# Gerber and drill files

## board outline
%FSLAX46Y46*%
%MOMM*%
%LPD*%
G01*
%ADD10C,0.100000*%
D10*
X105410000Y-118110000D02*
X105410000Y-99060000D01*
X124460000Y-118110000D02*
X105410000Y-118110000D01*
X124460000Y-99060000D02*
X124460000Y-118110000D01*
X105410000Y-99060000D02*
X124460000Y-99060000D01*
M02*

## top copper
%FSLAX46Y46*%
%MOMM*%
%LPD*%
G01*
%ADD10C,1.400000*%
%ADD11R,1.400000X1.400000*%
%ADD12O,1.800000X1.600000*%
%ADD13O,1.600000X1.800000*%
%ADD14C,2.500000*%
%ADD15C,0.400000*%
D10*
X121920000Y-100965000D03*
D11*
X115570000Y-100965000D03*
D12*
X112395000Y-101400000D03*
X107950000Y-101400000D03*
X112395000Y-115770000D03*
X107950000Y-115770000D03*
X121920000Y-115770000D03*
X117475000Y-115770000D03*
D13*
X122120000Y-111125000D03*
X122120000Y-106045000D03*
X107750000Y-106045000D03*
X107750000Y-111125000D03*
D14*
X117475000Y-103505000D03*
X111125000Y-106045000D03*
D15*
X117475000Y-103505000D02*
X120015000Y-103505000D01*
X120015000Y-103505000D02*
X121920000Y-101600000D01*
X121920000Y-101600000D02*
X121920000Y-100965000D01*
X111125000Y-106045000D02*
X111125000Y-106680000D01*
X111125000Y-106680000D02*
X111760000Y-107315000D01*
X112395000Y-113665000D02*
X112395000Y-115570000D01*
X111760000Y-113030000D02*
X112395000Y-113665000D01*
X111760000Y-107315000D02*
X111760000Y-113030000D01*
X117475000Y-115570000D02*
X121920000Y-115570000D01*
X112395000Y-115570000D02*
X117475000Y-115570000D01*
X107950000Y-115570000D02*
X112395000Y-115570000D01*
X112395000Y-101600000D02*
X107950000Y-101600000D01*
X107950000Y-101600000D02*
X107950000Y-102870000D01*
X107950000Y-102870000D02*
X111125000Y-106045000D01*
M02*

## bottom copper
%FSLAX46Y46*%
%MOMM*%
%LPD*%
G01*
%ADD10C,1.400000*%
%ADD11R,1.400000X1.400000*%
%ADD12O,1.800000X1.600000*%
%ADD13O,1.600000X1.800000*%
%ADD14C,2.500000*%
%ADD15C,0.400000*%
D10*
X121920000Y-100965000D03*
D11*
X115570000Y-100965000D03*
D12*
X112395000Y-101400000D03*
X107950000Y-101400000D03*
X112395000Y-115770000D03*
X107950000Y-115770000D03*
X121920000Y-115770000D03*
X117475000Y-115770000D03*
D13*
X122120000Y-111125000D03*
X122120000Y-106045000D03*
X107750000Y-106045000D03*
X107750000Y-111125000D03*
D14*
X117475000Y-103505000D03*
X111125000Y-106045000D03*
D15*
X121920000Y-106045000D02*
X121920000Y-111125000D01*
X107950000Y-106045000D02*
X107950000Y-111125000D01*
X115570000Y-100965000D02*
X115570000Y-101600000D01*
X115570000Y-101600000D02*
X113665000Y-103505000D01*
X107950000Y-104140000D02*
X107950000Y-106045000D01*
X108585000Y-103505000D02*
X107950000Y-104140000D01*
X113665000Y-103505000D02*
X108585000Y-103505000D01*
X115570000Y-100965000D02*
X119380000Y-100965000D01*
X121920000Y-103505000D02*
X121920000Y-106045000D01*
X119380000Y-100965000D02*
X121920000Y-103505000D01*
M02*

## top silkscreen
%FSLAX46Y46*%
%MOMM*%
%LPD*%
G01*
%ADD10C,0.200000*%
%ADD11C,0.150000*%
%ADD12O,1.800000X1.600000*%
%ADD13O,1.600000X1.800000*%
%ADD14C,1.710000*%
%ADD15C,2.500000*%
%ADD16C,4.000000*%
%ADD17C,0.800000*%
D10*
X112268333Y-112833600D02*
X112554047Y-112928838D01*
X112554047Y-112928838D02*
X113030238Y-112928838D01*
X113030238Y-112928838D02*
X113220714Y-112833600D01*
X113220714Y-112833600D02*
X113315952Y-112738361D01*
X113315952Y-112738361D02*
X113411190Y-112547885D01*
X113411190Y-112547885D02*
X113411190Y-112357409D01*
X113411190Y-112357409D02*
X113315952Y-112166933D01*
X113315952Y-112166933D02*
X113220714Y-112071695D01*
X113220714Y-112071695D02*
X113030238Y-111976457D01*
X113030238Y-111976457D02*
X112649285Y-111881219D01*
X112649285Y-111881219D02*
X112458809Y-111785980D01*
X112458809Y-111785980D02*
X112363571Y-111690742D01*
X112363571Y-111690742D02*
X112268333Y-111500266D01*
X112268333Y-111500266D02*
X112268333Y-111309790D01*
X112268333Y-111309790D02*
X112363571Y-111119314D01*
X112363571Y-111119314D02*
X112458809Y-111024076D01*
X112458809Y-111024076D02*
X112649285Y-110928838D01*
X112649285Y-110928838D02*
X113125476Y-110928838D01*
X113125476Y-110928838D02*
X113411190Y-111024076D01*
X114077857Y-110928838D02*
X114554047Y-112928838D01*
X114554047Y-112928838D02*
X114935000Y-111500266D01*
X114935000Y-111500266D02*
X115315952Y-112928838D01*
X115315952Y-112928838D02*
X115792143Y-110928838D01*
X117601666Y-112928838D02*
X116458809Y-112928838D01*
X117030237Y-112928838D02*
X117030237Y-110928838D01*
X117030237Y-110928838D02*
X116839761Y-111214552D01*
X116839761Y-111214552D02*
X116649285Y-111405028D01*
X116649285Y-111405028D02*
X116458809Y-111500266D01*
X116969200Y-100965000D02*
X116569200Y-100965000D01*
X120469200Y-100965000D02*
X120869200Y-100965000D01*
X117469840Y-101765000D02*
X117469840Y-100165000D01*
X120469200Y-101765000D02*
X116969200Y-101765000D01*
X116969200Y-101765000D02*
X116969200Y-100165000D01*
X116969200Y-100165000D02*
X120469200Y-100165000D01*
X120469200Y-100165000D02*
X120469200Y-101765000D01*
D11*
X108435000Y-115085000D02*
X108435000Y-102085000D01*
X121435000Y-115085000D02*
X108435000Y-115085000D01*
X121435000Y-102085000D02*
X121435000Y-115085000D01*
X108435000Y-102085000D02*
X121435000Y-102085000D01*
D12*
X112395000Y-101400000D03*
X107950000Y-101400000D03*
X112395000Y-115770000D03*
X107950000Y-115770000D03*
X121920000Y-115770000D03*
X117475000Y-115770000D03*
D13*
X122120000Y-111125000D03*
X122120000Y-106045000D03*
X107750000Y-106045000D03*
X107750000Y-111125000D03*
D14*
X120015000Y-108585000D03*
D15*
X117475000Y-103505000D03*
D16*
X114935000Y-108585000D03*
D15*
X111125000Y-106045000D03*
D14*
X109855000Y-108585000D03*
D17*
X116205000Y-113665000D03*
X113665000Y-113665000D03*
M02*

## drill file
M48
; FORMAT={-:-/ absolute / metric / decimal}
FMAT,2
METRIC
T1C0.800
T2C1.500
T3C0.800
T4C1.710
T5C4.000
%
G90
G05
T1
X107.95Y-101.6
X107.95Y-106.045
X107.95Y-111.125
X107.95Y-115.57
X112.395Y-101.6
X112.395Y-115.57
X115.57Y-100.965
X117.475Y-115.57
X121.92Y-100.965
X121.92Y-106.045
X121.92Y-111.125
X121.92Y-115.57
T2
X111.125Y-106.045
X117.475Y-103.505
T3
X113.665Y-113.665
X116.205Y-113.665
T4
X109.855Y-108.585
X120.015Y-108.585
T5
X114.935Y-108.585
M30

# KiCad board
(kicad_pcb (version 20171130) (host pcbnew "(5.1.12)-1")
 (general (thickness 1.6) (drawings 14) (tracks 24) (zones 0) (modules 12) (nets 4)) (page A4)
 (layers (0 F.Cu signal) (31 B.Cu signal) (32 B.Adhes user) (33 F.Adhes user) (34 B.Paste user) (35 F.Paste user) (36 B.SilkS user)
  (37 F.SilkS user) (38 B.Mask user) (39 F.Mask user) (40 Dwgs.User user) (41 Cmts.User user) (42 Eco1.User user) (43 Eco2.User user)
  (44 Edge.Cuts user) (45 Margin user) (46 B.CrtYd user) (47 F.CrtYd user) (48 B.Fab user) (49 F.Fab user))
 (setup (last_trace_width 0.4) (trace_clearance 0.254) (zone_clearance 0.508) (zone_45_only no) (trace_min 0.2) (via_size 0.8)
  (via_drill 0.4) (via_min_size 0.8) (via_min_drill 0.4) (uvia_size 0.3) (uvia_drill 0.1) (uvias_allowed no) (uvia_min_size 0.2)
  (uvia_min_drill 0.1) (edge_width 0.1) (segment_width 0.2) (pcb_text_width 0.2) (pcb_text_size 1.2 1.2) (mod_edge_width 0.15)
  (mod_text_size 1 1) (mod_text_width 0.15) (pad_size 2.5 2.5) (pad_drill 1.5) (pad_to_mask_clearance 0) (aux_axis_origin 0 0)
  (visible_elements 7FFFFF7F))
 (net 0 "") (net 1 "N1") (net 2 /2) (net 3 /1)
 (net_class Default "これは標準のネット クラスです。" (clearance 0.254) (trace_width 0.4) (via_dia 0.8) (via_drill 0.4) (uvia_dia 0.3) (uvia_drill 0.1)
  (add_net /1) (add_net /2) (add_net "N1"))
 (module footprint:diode (layer B.Cu) (at 115.57 100.965)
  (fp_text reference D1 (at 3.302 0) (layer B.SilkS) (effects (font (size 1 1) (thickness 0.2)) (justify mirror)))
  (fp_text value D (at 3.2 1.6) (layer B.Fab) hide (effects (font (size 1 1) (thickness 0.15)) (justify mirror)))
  (fp_line (start 1.3992 0) (end 0.9992 0) (layer F.SilkS) (width 0.2))
  (fp_line (start 4.8992 0) (end 5.2992 0) (layer F.SilkS) (width 0.2))
  (fp_line (start 1.89984 0.8) (end 1.89984 -0.8) (layer F.SilkS) (width 0.2))
  (fp_line (start 4.8992 0.8) (end 1.3992 0.8) (layer F.SilkS) (width 0.2))
  (fp_line (start 1.3992 0.8) (end 1.3992 -0.8) (layer F.SilkS) (width 0.2))
  (fp_line (start 1.3992 -0.8) (end 4.8992 -0.8) (layer F.SilkS) (width 0.2))
  (fp_line (start 4.8992 -0.8) (end 4.8992 0.8) (layer F.SilkS) (width 0.2))
  (pad 2 thru_hole circle (at 6.35 0) (size 1.4 1.4) (drill 0.8) (layers *.Cu *.Mask B.SilkS) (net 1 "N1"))
  (pad 1 thru_hole rect (at 0 0) (size 1.4 1.4) (drill 0.8) (layers *.Cu *.Mask B.SilkS) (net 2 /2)))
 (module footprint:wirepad (layer F.Cu) (at 112.395 101.6 180)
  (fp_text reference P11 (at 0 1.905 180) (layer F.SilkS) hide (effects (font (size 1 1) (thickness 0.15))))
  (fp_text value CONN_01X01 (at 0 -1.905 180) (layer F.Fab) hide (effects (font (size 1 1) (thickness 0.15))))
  (pad 1 thru_hole oval (at 0 0 180) (size 1.8 1.6) (drill 0.8 (offset 0 0.2)) (layers *.Cu *.Mask F.SilkS) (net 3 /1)))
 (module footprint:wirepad (layer F.Cu) (at 107.95 101.6 180)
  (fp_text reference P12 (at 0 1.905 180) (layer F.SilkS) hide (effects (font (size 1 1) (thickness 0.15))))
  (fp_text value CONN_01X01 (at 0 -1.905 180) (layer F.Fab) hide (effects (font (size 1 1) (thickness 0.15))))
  (pad 1 thru_hole oval (at 0 0 180) (size 1.8 1.6) (drill 0.8 (offset 0 0.2)) (layers *.Cu *.Mask F.SilkS) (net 3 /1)))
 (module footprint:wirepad (layer F.Cu) (at 112.395 115.57)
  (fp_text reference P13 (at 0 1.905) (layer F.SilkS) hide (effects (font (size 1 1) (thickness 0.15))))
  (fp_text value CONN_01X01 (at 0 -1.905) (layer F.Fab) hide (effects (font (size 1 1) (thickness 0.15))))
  (pad 1 thru_hole oval (at 0 0) (size 1.8 1.6) (drill 0.8 (offset 0 0.2)) (layers *.Cu *.Mask F.SilkS) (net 3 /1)))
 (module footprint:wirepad (layer F.Cu) (at 107.95 115.57)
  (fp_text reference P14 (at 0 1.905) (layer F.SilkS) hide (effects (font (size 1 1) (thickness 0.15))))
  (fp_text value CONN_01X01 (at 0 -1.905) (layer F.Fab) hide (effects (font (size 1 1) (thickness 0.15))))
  (pad 1 thru_hole oval (at 0 0) (size 1.8 1.6) (drill 0.8 (offset 0 0.2)) (layers *.Cu *.Mask F.SilkS) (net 3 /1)))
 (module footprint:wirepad (layer F.Cu) (at 121.92 115.57)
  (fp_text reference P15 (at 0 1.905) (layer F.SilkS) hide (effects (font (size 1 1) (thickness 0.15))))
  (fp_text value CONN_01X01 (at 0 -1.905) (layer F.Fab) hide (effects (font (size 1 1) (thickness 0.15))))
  (pad 1 thru_hole oval (at 0 0) (size 1.8 1.6) (drill 0.8 (offset 0 0.2)) (layers *.Cu *.Mask F.SilkS) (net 3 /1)))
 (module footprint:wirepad (layer F.Cu) (at 117.475 115.57)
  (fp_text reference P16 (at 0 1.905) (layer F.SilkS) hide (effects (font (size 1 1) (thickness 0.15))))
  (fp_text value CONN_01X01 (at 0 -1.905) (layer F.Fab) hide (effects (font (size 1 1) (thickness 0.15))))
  (pad 1 thru_hole oval (at 0 0) (size 1.8 1.6) (drill 0.8 (offset 0 0.2)) (layers *.Cu *.Mask F.SilkS) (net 3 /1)))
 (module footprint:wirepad (layer F.Cu) (at 121.92 111.125 90)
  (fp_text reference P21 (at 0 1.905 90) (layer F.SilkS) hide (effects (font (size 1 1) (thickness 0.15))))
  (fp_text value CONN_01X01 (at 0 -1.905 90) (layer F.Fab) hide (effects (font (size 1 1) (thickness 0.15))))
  (pad 1 thru_hole oval (at 0 0 90) (size 1.8 1.6) (drill 0.8 (offset 0 0.2)) (layers *.Cu *.Mask F.SilkS) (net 2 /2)))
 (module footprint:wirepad (layer F.Cu) (at 121.92 106.045 90)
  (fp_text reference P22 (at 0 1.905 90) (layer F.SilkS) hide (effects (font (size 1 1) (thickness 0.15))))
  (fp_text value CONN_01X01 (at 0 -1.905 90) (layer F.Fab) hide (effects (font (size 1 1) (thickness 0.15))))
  (pad 1 thru_hole oval (at 0 0 90) (size 1.8 1.6) (drill 0.8 (offset 0 0.2)) (layers *.Cu *.Mask F.SilkS) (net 2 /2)))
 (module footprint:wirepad (layer F.Cu) (at 107.95 106.045 270)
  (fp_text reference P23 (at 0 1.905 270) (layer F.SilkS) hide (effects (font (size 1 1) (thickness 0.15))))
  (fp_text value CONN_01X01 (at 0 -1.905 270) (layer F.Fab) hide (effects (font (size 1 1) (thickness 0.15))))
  (pad 1 thru_hole oval (at 0 0 270) (size 1.8 1.6) (drill 0.8 (offset 0 0.2)) (layers *.Cu *.Mask F.SilkS) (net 2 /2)))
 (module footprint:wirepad (layer F.Cu) (at 107.95 111.125 270)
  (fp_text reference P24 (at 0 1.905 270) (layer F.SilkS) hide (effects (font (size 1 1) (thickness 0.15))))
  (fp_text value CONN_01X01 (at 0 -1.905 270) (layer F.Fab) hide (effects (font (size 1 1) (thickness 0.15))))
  (pad 1 thru_hole oval (at 0 0 270) (size 1.8 1.6) (drill 0.8 (offset 0 0.2)) (layers *.Cu *.Mask F.SilkS) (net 2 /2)))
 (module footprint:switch (layer F.Cu) (at 114.935 108.585)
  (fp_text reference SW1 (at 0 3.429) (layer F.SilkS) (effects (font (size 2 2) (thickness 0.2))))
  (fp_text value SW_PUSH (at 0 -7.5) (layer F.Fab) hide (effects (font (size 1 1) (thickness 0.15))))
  (fp_line (start -6.5 6.5) (end -6.5 -6.5) (layer F.SilkS) (width 0.15))
  (fp_line (start 6.5 6.5) (end -6.5 6.5) (layer F.SilkS) (width 0.15))
  (fp_line (start 6.5 -6.5) (end 6.5 6.5) (layer F.SilkS) (width 0.15))
  (fp_line (start -6.5 -6.5) (end 6.5 -6.5) (layer F.SilkS) (width 0.15))
  (pad "" np_thru_hole circle (at 5.08 0) (size 1.71 1.71) (drill 1.71) (layers *.Cu *.Mask F.SilkS))
  (pad 2 thru_hole circle (at 2.54 -5.08) (size 2.5 2.5) (drill 1.5) (layers *.Cu *.Mask F.SilkS) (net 1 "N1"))
  (pad "" np_thru_hole circle (at 0 0) (size 4 4) (drill 4) (layers *.Cu *.Mask F.SilkS))
  (pad 1 thru_hole circle (at -3.81 -2.54) (size 2.5 2.5) (drill 1.5) (layers *.Cu *.Mask F.SilkS) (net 3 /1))
  (pad "" np_thru_hole circle (at -5.08 0) (size 1.71 1.71) (drill 1.71) (layers *.Cu *.Mask F.SilkS))
  (pad "" np_thru_hole circle (at 1.27 5.08) (size 0.8 0.8) (drill 0.8) (layers *.Cu *.Mask F.SilkS))
  (pad "" np_thru_hole circle (at -1.27 5.08) (size 0.8 0.8) (drill 0.8) (layers *.Cu *.Mask F.SilkS)))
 (gr_line (start 105.41 118.11) (end 105.41 99.06) (angle 90) (layer Edge.Cuts) (width 0.1))
 (gr_line (start 124.46 118.11) (end 105.41 118.11) (angle 90) (layer Edge.Cuts) (width 0.1))
 (gr_line (start 124.46 99.06) (end 124.46 118.11) (angle 90) (layer Edge.Cuts) (width 0.1))
 (gr_line (start 105.41 99.06) (end 124.46 99.06) (angle 90) (layer Edge.Cuts) (width 0.1))
 (segment (start 117.475 103.505) (end 120.015 103.505) (width 0.4) (layer F.Cu) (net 1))
 (segment (start 120.015 103.505) (end 121.92 101.6) (width 0.4) (layer F.Cu) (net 1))
 (segment (start 121.92 101.6) (end 121.92 100.965) (width 0.4) (layer F.Cu) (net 1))
 (segment (start 121.92 106.045) (end 121.92 111.125) (width 0.4) (layer B.Cu) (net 2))
 (segment (start 107.95 106.045) (end 107.95 111.125) (width 0.4) (layer B.Cu) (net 2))
 (segment (start 115.57 100.965) (end 115.57 101.6) (width 0.4) (layer B.Cu) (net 2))
 (segment (start 115.57 101.6) (end 113.665 103.505) (width 0.4) (layer B.Cu) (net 2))
 (segment (start 107.95 104.14) (end 107.95 106.045) (width 0.4) (layer B.Cu) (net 2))
 (segment (start 108.585 103.505) (end 107.95 104.14) (width 0.4) (layer B.Cu) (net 2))
 (segment (start 113.665 103.505) (end 108.585 103.505) (width 0.4) (layer B.Cu) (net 2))
 (segment (start 115.57 100.965) (end 119.38 100.965) (width 0.4) (layer B.Cu) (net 2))
 (segment (start 121.92 103.505) (end 121.92 106.045) (width 0.4) (layer B.Cu) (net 2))
 (segment (start 119.38 100.965) (end 121.92 103.505) (width 0.4) (layer B.Cu) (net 2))
 (segment (start 111.125 106.045) (end 111.125 106.68) (width 0.4) (layer F.Cu) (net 3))
 (segment (start 111.125 106.68) (end 111.76 107.315) (width 0.4) (layer F.Cu) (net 3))
 (segment (start 112.395 113.665) (end 112.395 115.57) (width 0.4) (layer F.Cu) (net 3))
 (segment (start 111.76 113.03) (end 112.395 113.665) (width 0.4) (layer F.Cu) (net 3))
 (segment (start 111.76 107.315) (end 111.76 113.03) (width 0.4) (layer F.Cu) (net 3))
 (segment (start 117.475 115.57) (end 121.92 115.57) (width 0.4) (layer F.Cu) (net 3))
 (segment (start 112.395 115.57) (end 117.475 115.57) (width 0.4) (layer F.Cu) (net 3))
 (segment (start 107.95 115.57) (end 112.395 115.57) (width 0.4) (layer F.Cu) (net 3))
 (segment (start 112.395 101.6) (end 107.95 101.6) (width 0.4) (layer F.Cu) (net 3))
 (segment (start 107.95 101.6) (end 107.95 102.87) (width 0.4) (layer F.Cu) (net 3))
 (segment (start 107.95 102.87) (end 111.125 106.045) (width 0.4) (layer F.Cu) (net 3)))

